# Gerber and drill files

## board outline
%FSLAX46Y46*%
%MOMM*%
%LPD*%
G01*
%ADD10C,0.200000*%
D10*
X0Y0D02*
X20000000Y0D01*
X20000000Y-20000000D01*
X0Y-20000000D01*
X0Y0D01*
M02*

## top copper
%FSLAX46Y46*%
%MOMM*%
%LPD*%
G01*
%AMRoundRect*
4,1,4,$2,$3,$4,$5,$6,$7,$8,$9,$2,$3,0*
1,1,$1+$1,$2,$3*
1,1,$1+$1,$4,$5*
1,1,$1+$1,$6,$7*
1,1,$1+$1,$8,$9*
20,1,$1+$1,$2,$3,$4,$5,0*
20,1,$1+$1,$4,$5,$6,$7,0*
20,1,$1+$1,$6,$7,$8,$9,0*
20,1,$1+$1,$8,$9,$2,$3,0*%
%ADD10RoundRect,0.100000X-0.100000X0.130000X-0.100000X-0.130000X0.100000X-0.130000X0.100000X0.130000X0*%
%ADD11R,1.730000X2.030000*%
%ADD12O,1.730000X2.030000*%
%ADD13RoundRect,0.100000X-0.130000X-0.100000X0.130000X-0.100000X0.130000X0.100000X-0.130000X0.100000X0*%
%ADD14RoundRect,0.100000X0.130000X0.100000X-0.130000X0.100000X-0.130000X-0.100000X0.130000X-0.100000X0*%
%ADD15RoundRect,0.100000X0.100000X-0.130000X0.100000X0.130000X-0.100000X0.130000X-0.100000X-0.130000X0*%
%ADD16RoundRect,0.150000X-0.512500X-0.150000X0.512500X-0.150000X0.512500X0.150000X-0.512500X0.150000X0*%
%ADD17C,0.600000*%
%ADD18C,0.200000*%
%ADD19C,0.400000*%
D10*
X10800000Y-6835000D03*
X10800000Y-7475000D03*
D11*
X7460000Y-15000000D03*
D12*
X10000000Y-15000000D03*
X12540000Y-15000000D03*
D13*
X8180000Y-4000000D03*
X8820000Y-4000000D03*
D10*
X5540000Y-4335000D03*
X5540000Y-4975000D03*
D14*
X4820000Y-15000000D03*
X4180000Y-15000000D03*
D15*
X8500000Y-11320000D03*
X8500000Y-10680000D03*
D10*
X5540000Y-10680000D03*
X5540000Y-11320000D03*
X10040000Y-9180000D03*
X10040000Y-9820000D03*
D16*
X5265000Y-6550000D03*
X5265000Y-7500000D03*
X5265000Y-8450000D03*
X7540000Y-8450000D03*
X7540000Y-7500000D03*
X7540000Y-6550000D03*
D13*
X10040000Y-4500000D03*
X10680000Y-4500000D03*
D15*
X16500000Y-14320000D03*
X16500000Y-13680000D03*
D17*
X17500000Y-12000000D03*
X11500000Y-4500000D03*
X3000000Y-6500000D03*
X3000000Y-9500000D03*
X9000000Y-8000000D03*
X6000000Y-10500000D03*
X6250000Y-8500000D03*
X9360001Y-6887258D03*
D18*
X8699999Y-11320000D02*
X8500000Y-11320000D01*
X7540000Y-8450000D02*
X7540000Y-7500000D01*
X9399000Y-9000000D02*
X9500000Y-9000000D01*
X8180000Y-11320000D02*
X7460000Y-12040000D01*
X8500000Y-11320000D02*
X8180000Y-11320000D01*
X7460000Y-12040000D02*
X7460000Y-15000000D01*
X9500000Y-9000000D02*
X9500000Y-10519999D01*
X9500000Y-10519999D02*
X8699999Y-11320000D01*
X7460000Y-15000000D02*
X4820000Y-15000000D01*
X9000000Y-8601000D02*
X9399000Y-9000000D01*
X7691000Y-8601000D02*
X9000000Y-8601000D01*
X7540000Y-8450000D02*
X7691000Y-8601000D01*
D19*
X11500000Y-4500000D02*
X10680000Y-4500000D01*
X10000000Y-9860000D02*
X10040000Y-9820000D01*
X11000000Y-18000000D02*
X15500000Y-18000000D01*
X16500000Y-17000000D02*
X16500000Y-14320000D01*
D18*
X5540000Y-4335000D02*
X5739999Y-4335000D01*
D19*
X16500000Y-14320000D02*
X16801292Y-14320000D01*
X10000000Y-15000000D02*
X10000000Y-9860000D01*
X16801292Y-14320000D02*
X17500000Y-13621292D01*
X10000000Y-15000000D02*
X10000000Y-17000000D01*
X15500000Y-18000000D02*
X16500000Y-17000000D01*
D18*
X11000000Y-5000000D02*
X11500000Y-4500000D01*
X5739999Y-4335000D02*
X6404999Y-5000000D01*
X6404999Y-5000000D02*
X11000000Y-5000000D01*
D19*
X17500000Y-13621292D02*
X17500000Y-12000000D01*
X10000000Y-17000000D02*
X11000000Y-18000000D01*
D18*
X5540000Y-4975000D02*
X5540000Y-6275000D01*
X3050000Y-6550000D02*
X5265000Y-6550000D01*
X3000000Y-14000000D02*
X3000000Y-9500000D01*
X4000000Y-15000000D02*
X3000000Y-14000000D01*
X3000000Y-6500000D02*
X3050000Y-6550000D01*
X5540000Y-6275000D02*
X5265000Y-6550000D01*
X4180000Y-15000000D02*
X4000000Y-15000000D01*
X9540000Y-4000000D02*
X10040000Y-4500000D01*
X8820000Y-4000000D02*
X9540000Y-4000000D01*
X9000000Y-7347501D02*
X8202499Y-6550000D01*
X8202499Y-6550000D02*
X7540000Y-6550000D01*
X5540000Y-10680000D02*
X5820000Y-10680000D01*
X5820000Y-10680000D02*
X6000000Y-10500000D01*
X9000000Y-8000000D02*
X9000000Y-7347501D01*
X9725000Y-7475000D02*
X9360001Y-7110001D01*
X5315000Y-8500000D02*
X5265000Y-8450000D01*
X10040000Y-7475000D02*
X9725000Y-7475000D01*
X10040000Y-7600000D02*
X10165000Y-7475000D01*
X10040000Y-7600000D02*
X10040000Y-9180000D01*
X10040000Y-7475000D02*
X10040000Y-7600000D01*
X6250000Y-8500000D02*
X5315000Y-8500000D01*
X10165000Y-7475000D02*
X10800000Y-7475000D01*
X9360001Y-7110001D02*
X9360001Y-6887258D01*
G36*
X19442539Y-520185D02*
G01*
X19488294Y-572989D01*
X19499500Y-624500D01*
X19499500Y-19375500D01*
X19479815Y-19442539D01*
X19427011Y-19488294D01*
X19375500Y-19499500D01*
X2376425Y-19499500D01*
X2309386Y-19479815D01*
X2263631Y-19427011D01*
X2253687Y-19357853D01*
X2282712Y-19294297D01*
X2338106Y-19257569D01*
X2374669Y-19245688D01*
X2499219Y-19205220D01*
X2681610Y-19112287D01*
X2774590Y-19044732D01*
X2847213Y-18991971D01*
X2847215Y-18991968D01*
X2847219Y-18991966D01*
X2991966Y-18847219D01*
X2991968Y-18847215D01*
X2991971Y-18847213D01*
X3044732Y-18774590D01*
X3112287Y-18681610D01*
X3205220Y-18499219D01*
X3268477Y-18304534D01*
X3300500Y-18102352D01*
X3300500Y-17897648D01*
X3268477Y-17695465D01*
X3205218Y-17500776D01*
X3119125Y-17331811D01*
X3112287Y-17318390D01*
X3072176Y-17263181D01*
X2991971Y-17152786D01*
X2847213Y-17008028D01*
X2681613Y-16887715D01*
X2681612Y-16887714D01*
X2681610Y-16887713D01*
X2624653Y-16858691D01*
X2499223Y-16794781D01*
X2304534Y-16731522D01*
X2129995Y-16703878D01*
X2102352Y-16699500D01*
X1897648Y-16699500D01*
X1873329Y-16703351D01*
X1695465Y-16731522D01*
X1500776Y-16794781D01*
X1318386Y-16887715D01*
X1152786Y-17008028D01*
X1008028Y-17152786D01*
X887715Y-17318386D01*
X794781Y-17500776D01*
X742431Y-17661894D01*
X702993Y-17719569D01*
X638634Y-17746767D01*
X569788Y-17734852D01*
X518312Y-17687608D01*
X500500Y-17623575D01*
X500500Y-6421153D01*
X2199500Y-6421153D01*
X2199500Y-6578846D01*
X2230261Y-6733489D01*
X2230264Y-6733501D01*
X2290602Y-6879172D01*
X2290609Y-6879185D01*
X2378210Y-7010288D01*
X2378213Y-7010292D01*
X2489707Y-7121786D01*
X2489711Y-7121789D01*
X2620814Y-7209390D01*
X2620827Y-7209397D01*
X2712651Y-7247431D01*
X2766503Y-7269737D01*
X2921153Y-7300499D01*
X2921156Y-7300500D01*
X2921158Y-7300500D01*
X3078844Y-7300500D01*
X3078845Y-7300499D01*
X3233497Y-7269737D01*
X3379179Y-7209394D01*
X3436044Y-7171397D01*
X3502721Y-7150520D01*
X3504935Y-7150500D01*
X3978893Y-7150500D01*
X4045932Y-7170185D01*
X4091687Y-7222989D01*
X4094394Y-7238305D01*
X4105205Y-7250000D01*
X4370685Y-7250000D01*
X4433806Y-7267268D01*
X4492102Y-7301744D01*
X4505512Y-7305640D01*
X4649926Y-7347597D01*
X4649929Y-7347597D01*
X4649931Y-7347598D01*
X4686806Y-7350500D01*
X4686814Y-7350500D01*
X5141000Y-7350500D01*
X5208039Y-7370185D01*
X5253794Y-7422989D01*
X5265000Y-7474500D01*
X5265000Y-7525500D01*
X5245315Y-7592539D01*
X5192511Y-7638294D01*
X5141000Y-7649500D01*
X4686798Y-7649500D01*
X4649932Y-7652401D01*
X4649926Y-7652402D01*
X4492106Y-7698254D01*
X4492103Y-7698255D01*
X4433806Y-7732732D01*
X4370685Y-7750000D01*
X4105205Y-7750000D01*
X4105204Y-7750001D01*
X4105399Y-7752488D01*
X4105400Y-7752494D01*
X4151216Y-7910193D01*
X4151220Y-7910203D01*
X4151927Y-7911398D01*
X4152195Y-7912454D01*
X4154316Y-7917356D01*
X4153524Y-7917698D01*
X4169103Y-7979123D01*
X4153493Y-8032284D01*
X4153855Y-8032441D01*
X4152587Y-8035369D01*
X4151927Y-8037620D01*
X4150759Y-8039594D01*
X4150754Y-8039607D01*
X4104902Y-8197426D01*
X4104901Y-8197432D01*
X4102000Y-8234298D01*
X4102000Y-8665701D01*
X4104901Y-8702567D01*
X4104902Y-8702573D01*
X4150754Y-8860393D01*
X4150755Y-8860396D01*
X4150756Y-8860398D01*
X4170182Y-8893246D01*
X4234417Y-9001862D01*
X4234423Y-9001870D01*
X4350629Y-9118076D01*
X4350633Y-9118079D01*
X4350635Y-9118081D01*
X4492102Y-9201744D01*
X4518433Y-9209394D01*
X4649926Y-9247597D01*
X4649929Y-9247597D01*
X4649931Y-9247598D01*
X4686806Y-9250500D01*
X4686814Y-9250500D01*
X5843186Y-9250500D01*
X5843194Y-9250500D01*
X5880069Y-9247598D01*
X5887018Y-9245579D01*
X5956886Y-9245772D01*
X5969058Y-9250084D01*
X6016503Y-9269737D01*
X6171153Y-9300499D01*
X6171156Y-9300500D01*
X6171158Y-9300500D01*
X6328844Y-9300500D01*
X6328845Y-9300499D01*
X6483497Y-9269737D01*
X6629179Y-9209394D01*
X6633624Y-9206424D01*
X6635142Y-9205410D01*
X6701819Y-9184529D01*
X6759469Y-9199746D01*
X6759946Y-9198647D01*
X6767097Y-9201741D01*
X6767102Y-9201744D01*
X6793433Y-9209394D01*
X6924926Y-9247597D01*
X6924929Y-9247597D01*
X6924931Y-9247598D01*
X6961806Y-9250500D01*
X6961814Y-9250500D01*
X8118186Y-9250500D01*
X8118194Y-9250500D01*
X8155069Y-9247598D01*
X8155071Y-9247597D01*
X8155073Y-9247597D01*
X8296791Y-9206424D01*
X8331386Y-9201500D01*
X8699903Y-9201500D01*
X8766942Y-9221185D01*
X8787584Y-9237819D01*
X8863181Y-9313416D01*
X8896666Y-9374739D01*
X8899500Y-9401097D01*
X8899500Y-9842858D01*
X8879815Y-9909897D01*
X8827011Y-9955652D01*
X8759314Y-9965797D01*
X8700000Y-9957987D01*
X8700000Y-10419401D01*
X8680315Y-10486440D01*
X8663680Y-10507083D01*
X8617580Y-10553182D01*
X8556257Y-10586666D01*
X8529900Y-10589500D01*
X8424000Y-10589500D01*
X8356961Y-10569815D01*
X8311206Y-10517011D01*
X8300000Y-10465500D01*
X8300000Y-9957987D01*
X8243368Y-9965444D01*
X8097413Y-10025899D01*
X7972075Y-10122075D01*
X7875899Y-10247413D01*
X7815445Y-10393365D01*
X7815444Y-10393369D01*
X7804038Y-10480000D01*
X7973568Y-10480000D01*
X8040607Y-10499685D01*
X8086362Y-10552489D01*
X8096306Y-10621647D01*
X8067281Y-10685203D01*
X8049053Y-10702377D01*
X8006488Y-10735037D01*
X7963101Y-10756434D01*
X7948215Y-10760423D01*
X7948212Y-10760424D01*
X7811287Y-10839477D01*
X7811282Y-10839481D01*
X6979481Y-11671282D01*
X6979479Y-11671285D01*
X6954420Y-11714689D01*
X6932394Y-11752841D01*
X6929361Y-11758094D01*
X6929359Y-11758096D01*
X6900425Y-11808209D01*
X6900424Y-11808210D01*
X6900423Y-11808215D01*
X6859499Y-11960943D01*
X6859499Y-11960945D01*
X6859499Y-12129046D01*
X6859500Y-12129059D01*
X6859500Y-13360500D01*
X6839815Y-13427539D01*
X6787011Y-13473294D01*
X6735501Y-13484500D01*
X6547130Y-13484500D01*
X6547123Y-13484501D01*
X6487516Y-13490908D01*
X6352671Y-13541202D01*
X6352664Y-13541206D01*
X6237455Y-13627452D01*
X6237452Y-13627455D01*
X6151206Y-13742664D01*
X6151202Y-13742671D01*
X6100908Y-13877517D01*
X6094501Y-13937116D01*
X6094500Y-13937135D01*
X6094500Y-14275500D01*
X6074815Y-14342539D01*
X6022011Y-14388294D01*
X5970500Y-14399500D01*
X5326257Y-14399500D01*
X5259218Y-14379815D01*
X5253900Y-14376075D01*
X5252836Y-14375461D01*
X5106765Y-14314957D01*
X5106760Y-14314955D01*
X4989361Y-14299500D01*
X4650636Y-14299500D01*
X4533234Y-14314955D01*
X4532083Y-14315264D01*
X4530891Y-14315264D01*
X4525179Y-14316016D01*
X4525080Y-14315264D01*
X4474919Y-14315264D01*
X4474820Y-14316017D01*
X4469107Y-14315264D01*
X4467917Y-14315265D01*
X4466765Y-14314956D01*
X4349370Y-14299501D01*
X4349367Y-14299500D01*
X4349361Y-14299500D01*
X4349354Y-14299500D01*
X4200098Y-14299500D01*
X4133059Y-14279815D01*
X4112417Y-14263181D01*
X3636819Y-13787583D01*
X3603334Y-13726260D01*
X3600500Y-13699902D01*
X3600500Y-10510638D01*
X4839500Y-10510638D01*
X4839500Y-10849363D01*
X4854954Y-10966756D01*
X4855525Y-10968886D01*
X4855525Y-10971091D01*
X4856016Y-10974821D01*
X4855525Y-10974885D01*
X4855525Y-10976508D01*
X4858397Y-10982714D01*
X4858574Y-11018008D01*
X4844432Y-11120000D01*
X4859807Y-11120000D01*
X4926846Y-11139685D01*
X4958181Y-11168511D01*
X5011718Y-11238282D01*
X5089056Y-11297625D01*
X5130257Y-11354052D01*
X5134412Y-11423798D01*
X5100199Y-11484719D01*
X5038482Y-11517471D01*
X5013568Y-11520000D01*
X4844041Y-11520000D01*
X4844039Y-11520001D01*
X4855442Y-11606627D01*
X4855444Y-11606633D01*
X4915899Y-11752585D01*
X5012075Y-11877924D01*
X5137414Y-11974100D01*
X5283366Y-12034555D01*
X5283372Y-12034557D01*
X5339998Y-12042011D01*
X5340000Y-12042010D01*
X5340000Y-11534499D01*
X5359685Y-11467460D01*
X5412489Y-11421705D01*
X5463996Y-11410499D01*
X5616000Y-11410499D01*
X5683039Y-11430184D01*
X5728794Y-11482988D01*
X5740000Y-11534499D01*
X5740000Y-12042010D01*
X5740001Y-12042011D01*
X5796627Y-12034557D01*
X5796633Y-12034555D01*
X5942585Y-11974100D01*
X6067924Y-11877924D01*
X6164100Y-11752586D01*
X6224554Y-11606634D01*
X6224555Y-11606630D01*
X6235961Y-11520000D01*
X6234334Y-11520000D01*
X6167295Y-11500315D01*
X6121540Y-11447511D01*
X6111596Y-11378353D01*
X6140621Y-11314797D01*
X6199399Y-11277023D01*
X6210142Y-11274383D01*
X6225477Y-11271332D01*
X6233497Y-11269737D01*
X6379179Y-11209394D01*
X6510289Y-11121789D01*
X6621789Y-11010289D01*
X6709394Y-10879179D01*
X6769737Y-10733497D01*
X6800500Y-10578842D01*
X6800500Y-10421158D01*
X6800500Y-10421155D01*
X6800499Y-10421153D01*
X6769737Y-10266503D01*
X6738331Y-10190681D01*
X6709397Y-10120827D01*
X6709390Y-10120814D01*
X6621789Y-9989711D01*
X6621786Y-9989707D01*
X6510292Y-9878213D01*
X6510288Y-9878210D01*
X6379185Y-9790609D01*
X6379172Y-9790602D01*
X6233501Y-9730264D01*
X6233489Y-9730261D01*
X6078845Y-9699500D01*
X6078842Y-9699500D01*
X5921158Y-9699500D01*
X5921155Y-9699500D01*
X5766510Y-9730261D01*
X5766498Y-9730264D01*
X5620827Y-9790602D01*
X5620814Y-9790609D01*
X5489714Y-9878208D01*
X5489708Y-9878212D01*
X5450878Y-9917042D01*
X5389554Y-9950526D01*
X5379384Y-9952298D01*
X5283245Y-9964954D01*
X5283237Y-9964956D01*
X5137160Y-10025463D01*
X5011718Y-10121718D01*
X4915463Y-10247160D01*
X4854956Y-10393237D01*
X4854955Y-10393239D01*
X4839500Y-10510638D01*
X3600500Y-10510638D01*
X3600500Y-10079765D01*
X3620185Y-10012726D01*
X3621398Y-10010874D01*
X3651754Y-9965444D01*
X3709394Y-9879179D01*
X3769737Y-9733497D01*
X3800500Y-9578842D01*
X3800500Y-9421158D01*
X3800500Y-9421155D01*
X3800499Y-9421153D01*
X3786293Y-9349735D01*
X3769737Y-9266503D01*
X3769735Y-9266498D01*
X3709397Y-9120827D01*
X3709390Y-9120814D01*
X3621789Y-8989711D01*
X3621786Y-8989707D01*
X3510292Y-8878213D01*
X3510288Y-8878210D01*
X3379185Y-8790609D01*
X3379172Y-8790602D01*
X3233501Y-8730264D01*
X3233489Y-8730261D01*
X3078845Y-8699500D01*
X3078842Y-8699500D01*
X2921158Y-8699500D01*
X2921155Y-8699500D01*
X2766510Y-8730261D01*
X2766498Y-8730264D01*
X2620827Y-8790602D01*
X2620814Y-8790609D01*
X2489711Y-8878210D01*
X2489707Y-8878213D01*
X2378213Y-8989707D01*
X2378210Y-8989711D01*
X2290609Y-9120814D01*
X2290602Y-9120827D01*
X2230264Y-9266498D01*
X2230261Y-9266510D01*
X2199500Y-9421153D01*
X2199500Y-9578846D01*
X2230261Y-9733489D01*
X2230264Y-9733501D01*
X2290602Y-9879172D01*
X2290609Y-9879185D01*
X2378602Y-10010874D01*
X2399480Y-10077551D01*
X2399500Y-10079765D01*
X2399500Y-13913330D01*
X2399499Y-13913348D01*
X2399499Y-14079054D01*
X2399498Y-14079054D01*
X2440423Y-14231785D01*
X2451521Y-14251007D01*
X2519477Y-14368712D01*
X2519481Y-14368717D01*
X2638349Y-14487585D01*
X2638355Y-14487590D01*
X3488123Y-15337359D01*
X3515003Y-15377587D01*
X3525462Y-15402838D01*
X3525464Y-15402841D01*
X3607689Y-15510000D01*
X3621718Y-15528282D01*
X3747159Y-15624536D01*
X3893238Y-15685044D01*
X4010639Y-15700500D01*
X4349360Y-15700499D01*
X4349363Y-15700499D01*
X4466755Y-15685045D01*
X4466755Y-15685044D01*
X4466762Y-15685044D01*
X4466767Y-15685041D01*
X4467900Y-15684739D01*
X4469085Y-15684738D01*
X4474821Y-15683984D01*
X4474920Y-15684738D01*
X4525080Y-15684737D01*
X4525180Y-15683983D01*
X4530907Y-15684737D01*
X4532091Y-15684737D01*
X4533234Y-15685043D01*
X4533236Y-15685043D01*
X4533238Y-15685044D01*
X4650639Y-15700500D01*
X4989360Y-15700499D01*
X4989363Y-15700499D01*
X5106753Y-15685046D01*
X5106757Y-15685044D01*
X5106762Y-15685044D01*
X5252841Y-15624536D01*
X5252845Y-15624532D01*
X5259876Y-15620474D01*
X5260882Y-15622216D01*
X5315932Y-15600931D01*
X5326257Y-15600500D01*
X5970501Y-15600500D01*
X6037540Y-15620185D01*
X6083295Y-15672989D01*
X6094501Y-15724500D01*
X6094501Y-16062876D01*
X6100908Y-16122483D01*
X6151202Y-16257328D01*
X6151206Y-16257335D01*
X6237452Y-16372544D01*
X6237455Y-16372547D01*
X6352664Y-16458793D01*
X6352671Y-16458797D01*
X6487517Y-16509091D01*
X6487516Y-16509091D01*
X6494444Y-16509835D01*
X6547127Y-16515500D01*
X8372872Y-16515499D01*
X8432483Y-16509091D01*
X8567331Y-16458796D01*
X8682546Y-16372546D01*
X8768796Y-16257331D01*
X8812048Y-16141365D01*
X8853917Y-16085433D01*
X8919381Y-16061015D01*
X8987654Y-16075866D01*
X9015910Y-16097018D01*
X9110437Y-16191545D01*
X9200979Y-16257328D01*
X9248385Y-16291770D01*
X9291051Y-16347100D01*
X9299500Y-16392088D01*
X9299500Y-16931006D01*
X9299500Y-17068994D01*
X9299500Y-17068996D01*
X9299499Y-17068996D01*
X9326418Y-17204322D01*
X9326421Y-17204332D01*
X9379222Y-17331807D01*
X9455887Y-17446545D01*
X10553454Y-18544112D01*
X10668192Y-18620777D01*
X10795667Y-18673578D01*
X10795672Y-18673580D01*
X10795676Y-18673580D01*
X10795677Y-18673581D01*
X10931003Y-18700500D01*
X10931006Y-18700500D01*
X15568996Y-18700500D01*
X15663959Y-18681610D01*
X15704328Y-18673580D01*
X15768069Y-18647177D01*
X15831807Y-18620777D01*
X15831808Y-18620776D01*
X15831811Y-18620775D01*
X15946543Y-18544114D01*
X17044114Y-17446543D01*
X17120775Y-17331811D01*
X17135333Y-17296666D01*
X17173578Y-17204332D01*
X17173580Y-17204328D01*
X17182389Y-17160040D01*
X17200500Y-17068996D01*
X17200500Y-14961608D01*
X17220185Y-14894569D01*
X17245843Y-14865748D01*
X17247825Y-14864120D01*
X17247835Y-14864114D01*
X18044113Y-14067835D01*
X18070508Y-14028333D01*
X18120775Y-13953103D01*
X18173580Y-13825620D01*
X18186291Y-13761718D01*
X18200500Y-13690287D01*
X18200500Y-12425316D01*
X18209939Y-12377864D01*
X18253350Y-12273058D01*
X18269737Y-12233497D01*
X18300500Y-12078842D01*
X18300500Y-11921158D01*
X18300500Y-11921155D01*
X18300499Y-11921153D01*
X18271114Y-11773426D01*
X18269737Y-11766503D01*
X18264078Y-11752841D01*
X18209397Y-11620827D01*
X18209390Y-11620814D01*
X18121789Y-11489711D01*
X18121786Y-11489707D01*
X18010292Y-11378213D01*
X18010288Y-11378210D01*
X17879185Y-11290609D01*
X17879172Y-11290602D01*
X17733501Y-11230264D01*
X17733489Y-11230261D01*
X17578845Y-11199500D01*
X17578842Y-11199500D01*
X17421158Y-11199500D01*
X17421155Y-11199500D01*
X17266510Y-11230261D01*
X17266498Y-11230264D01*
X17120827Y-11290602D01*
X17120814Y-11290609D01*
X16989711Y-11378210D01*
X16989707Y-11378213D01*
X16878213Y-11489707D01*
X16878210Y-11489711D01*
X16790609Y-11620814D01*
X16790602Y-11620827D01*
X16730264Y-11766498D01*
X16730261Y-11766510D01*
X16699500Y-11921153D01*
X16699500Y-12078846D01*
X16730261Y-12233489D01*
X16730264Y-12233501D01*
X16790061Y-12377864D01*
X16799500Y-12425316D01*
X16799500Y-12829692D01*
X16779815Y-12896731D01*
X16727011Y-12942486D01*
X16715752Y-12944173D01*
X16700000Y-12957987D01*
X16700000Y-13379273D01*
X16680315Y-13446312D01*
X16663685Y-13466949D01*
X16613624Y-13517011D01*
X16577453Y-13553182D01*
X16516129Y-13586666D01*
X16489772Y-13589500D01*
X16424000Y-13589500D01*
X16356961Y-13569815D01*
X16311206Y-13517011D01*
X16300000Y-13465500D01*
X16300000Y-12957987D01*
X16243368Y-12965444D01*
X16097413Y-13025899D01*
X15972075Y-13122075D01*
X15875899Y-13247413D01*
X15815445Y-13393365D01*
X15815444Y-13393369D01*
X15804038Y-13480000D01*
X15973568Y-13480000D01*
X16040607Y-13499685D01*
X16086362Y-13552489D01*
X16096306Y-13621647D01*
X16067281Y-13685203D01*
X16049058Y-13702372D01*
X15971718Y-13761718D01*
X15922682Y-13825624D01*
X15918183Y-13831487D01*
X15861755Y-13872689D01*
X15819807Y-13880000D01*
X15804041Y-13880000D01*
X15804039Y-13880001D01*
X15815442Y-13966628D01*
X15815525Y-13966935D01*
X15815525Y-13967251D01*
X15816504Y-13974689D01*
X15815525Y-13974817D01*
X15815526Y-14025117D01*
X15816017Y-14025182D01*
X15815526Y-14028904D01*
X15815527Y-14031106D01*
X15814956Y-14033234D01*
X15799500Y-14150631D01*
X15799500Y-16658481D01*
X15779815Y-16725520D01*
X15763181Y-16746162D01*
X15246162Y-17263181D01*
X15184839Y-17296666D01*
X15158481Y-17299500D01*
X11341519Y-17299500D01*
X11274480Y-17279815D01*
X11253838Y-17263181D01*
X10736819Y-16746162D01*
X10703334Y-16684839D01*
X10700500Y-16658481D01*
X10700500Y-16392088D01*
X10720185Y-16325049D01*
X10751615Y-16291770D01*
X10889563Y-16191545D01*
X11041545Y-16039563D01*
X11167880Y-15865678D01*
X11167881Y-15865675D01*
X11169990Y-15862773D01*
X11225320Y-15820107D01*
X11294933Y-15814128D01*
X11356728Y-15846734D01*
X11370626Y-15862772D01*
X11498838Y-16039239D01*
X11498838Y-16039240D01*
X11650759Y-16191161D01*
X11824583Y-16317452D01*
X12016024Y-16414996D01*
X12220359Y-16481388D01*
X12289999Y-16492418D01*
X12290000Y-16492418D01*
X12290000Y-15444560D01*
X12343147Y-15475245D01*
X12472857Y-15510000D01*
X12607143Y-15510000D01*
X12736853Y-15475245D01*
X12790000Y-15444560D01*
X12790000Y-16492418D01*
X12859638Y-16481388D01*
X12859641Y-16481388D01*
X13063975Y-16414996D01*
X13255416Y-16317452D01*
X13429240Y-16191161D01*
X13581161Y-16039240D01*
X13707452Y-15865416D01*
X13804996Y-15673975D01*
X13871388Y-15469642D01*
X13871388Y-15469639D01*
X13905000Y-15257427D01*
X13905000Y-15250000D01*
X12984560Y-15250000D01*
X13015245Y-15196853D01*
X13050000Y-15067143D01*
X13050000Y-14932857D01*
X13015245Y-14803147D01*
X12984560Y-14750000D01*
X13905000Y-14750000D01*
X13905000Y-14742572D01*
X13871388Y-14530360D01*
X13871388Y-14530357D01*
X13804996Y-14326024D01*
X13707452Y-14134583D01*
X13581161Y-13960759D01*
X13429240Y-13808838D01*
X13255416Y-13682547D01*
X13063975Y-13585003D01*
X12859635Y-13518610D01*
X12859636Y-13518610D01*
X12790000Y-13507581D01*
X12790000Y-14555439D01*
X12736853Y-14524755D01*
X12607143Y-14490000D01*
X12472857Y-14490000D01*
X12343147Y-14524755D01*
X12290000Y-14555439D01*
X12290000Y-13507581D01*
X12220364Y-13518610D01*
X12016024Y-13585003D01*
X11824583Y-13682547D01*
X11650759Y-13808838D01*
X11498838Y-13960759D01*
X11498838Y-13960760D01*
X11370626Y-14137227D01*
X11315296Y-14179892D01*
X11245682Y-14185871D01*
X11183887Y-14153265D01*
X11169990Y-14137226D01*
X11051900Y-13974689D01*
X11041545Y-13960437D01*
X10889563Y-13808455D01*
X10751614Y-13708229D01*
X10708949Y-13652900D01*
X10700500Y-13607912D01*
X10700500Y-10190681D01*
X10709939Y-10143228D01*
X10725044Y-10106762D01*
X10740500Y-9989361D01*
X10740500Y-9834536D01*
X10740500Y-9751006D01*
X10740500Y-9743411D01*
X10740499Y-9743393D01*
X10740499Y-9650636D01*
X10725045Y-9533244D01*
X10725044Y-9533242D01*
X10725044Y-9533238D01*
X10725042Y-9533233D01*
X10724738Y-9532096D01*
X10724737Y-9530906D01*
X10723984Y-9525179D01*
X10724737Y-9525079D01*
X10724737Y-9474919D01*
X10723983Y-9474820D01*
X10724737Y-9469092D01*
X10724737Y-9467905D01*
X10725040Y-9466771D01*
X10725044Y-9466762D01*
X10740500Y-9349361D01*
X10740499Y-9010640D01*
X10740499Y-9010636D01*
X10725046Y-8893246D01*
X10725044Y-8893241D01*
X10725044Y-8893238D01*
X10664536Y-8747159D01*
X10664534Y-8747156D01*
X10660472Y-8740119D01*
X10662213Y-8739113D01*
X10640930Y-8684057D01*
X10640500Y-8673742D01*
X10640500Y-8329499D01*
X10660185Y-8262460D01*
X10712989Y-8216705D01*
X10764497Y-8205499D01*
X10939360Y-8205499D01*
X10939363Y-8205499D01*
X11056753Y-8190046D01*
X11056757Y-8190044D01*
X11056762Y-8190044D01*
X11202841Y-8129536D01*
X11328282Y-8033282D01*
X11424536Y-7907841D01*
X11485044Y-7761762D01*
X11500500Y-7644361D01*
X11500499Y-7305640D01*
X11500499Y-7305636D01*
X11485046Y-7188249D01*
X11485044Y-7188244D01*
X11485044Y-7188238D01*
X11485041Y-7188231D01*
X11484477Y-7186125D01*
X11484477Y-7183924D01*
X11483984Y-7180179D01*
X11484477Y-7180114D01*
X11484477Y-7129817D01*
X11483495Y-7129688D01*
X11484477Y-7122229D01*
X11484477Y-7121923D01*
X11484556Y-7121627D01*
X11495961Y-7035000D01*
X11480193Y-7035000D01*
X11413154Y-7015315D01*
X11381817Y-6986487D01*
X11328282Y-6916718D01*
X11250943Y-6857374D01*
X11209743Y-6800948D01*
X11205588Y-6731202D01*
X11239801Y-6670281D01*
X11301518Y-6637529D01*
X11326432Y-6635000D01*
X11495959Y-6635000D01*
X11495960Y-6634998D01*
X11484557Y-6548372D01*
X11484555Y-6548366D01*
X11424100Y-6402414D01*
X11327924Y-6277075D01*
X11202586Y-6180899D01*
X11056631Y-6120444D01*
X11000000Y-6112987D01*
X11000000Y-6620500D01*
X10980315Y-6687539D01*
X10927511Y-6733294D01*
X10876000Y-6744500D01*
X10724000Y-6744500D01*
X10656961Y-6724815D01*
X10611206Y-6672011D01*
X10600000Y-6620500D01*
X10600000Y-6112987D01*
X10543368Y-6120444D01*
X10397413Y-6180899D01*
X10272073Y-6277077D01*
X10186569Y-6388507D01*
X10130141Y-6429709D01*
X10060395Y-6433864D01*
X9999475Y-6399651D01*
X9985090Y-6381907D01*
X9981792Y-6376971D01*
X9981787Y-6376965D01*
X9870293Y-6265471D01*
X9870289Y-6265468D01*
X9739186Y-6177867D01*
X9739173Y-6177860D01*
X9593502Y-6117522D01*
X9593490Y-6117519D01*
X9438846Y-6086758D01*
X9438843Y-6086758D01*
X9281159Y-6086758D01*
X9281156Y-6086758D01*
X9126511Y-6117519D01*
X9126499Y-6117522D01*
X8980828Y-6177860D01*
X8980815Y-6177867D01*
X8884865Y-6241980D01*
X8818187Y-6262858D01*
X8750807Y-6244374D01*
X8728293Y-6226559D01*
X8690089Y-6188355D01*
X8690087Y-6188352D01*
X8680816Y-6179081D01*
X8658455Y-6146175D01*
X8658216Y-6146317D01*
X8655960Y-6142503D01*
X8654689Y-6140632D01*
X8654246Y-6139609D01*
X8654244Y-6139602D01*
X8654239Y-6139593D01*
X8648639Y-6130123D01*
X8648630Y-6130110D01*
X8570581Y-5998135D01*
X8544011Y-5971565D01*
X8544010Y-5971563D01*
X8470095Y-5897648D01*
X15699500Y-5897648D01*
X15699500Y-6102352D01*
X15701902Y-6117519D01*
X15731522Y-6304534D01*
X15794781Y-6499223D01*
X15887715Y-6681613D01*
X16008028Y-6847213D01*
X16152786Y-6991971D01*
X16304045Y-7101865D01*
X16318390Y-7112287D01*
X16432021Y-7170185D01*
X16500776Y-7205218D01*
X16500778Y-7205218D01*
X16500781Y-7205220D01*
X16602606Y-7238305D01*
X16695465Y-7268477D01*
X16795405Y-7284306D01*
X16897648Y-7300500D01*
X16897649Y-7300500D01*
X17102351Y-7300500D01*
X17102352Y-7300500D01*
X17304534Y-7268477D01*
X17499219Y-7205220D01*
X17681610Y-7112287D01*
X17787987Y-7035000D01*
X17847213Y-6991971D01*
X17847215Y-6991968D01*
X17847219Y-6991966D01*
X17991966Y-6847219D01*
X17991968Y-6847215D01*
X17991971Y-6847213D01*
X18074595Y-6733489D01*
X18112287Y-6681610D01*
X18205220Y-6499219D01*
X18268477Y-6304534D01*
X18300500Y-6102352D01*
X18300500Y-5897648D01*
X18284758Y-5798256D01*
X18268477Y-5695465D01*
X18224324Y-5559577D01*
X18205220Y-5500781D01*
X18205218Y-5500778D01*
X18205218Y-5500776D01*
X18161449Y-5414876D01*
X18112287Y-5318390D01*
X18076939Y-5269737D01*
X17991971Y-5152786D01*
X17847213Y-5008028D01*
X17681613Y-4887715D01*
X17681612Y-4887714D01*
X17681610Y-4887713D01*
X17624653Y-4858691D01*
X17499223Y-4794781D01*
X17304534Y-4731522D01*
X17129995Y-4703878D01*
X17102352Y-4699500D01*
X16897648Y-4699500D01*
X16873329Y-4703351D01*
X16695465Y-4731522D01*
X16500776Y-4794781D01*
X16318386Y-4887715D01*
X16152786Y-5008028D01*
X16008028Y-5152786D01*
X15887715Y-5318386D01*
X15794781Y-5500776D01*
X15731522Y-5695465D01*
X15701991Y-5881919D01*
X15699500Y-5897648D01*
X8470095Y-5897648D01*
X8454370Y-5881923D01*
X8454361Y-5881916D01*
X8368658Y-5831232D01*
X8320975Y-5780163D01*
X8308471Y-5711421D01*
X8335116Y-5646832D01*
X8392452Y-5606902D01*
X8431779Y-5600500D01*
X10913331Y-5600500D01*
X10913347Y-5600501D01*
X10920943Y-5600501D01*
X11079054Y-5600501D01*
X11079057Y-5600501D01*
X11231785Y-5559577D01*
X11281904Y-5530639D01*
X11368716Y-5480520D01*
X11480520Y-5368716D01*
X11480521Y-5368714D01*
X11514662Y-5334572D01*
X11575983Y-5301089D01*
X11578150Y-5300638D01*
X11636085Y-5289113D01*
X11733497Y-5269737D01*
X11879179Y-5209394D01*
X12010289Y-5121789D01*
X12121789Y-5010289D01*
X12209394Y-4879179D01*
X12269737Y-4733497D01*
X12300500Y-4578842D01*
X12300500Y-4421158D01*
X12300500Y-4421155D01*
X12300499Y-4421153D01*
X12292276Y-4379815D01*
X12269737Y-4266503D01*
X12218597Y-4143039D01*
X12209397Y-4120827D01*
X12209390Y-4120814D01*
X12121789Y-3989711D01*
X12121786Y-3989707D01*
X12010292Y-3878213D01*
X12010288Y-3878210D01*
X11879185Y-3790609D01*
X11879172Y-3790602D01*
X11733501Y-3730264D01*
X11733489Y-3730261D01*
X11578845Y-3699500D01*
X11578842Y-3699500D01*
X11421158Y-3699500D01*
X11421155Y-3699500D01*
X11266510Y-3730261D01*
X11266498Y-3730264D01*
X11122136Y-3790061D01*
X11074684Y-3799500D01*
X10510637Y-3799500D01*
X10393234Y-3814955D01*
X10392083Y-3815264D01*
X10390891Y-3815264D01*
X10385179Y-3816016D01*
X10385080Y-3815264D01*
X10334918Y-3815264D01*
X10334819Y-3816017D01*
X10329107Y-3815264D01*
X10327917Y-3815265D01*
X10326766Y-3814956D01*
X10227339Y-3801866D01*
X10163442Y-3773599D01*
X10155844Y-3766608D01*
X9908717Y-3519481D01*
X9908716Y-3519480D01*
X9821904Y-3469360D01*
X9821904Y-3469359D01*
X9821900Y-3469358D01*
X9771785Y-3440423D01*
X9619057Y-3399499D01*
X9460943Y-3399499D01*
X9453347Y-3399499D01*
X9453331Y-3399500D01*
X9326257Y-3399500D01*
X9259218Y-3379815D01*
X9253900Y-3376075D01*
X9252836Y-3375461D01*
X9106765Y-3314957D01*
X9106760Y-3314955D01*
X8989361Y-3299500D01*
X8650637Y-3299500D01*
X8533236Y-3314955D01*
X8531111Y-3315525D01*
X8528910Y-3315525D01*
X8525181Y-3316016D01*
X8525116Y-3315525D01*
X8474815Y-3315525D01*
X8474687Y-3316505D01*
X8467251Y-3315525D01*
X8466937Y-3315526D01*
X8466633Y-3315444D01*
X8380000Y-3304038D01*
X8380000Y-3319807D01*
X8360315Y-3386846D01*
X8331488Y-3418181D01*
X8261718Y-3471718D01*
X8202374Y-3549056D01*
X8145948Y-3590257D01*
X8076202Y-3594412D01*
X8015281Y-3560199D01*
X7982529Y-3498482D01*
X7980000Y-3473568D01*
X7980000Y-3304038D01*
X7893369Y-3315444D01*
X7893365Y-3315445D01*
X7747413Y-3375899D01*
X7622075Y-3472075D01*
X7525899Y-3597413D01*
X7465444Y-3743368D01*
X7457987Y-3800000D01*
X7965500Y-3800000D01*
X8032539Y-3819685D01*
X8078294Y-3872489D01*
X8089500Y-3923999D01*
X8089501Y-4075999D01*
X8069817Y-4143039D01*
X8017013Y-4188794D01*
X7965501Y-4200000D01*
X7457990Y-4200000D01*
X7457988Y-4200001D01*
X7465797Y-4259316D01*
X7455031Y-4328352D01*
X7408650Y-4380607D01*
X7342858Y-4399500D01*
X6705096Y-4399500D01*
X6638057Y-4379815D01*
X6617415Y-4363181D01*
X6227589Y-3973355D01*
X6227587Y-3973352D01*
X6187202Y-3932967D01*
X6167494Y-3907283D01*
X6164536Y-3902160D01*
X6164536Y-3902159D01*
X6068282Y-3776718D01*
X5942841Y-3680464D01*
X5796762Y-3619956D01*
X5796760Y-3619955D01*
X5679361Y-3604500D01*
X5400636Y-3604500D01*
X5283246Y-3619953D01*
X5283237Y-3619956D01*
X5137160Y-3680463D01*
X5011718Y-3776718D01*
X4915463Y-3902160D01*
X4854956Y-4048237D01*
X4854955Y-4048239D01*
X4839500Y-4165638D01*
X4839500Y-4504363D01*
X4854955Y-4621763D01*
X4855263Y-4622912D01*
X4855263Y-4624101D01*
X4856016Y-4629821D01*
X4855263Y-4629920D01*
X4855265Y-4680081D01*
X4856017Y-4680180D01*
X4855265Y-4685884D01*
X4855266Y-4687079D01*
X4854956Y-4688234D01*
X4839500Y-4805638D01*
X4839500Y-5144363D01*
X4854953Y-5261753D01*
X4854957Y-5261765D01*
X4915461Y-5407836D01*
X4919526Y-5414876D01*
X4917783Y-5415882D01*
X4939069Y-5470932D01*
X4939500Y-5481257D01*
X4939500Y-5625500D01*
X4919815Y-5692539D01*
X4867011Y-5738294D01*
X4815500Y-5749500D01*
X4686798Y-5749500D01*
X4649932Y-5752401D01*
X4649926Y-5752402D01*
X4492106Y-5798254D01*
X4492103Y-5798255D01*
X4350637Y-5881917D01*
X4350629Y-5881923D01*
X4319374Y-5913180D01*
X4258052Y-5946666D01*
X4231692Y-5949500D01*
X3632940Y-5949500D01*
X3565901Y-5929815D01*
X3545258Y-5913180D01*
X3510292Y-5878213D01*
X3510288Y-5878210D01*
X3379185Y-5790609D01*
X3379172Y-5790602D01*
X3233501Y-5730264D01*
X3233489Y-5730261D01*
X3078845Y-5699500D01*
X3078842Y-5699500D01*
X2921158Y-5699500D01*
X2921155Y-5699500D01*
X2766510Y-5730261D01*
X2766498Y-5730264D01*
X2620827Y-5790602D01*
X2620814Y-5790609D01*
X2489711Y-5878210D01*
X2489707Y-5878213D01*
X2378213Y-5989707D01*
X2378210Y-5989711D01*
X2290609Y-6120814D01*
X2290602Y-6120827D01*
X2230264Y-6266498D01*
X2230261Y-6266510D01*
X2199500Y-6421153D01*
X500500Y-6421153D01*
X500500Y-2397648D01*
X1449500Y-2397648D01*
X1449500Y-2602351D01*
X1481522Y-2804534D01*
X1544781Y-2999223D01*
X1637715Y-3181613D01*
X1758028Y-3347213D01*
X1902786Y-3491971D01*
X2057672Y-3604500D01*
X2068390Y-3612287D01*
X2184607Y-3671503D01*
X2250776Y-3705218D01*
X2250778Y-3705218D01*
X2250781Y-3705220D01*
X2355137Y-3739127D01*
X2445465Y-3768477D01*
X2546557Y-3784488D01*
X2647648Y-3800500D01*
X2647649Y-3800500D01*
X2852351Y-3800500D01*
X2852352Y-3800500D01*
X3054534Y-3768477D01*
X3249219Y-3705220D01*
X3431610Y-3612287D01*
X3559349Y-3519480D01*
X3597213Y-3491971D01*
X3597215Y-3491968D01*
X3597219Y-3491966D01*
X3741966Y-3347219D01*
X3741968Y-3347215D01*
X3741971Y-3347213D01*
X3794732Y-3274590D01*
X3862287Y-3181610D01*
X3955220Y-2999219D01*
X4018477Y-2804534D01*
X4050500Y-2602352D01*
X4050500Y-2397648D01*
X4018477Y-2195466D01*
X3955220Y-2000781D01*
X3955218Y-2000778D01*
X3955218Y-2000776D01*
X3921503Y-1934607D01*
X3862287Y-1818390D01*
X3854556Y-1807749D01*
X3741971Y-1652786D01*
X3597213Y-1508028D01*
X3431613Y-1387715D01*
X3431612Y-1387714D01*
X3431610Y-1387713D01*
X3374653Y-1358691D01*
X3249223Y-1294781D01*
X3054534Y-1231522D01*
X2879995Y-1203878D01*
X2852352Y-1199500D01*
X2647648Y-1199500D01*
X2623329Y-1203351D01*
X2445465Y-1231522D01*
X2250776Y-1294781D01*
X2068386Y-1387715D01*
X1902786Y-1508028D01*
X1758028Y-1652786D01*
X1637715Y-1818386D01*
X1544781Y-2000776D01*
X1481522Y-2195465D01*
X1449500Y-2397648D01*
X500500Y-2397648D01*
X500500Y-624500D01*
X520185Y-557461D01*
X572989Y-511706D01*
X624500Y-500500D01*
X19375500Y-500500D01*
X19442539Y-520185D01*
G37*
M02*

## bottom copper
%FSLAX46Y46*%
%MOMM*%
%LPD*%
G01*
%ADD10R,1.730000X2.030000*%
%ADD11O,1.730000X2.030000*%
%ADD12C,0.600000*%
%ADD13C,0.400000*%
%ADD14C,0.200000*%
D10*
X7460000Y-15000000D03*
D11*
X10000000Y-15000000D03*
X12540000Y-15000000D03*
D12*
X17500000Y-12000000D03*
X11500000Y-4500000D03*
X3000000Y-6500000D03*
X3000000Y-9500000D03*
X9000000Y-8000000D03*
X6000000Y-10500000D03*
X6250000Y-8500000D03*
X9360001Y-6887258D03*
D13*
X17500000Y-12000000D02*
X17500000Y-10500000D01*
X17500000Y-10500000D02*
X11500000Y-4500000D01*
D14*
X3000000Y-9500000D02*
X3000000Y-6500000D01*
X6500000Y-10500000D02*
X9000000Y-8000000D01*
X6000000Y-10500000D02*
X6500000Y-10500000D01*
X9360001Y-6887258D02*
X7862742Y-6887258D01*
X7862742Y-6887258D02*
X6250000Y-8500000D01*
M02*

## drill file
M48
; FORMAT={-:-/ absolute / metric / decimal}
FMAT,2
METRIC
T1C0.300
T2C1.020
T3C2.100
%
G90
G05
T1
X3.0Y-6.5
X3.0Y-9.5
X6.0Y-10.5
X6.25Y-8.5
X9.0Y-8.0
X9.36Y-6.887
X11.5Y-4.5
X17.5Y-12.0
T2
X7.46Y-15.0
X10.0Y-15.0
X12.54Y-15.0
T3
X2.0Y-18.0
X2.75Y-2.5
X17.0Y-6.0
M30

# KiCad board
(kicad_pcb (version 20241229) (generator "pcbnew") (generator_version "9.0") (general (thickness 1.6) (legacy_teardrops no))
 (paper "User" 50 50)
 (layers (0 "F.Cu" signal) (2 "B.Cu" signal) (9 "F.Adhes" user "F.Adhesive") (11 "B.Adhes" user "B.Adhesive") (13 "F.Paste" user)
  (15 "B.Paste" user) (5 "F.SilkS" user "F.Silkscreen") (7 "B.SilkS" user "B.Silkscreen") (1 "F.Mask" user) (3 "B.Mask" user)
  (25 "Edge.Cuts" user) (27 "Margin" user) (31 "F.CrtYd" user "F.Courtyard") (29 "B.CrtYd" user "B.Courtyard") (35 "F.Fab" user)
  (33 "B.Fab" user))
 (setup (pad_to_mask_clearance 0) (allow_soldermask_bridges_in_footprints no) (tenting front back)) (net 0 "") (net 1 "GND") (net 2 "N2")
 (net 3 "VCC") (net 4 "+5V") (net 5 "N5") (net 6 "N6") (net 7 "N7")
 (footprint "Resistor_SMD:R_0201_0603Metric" (layer "F.Cu") (at 10.8 7.155 -90)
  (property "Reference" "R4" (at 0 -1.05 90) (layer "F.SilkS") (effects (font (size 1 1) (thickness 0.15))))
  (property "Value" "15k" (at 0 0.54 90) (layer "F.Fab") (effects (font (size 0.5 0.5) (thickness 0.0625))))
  (pad "" smd roundrect (at -0.345 0 270) (size 0.318 0.36) (layers "F.Paste") (roundrect_rratio 0.25))
  (pad "" smd roundrect (at 0.345 0 270) (size 0.318 0.36) (layers "F.Paste") (roundrect_rratio 0.25))
  (pad "1" smd roundrect (at -0.32 0 270) (size 0.46 0.4) (layers "F.Cu" "F.Mask") (roundrect_rratio 0.25) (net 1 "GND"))
  (pad "2" smd roundrect (at 0.32 0 270) (size 0.46 0.4) (layers "F.Cu" "F.Mask") (roundrect_rratio 0.25) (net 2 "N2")))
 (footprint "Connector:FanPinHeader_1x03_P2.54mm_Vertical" (layer "F.Cu") (at 7.46 15)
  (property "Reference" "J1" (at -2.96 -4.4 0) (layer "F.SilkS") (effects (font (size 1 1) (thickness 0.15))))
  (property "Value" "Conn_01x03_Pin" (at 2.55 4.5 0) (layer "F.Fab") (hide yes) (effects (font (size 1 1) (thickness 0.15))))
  (pad "1" thru_hole rect (at 0 0 90) (size 2.03 1.73) (drill 1.02) (layers "*.Cu" "*.Mask") (remove_unused_layers no) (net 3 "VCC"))
  (pad "2" thru_hole oval (at 2.54 0 90) (size 2.03 1.73) (drill 1.02) (layers "*.Cu" "*.Mask") (remove_unused_layers no) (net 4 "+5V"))
  (pad "3" thru_hole oval (at 5.08 0 90) (size 2.03 1.73) (drill 1.02) (layers "*.Cu" "*.Mask") (remove_unused_layers no) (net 1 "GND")))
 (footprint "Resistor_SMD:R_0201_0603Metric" (layer "F.Cu") (at 8.5 4)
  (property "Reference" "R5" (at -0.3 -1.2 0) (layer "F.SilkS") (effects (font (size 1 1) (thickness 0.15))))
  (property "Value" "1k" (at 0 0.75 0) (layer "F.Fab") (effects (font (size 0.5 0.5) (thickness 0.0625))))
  (pad "" smd roundrect (at -0.345 0) (size 0.318 0.36) (layers "F.Paste") (roundrect_rratio 0.25))
  (pad "" smd roundrect (at 0.345 0) (size 0.318 0.36) (layers "F.Paste") (roundrect_rratio 0.25))
  (pad "1" smd roundrect (at -0.32 0) (size 0.46 0.4) (layers "F.Cu" "F.Mask") (roundrect_rratio 0.25) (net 1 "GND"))
  (pad "2" smd roundrect (at 0.32 0) (size 0.46 0.4) (layers "F.Cu" "F.Mask") (roundrect_rratio 0.25) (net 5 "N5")))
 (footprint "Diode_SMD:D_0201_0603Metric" (layer "F.Cu") (at 5.54 4.655 -90)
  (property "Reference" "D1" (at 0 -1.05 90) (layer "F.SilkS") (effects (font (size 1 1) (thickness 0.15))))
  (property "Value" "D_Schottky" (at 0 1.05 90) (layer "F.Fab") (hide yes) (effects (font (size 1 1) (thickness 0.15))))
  (pad "" smd roundrect (at -0.345 0 270) (size 0.318 0.36) (layers "F.Paste") (roundrect_rratio 0.25))
  (pad "" smd roundrect (at 0.345 0 270) (size 0.318 0.36) (layers "F.Paste") (roundrect_rratio 0.25))
  (pad "1" smd roundrect (at -0.32 0 270) (size 0.46 0.4) (layers "F.Cu" "F.Mask") (roundrect_rratio 0.25) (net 4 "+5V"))
  (pad "2" smd roundrect (at 0.32 0 270) (size 0.46 0.4) (layers "F.Cu" "F.Mask") (roundrect_rratio 0.25) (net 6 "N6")))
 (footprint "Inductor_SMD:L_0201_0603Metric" (layer "F.Cu") (at 4.5 15 180)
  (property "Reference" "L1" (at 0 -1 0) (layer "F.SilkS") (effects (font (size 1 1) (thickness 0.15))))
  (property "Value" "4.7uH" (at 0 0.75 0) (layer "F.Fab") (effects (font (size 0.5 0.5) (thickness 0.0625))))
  (pad "" smd roundrect (at -0.345 0 180) (size 0.318 0.36) (layers "F.Paste") (roundrect_rratio 0.25))
  (pad "" smd roundrect (at 0.345 0 180) (size 0.318 0.36) (layers "F.Paste") (roundrect_rratio 0.25))
  (pad "1" smd roundrect (at -0.32 0 180) (size 0.46 0.4) (layers "F.Cu" "F.Mask") (roundrect_rratio 0.25) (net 3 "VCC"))
  (pad "2" smd roundrect (at 0.32 0 180) (size 0.46 0.4) (layers "F.Cu" "F.Mask") (roundrect_rratio 0.25) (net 6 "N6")))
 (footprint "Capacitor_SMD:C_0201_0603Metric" (layer "F.Cu") (at 8.5 11 90)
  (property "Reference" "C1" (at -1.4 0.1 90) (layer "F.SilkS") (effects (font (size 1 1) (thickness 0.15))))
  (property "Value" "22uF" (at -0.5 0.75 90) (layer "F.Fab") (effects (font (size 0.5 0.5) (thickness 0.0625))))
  (pad "" smd roundrect (at -0.345 0 90) (size 0.318 0.36) (layers "F.Paste") (roundrect_rratio 0.25))
  (pad "" smd roundrect (at 0.345 0 90) (size 0.318 0.36) (layers "F.Paste") (roundrect_rratio 0.25))
  (pad "1" smd roundrect (at -0.32 0 90) (size 0.46 0.4) (layers "F.Cu" "F.Mask") (roundrect_rratio 0.25) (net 3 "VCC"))
  (pad "2" smd roundrect (at 0.32 0 90) (size 0.46 0.4) (layers "F.Cu" "F.Mask") (roundrect_rratio 0.25) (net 1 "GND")))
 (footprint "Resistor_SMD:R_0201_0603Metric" (layer "F.Cu") (at 5.54 11 -90)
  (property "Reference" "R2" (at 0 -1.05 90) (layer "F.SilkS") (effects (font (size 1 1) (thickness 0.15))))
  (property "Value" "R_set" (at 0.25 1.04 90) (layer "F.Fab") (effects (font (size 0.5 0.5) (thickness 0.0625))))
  (pad "" smd roundrect (at -0.345 0 270) (size 0.318 0.36) (layers "F.Paste") (roundrect_rratio 0.25))
  (pad "" smd roundrect (at 0.345 0 270) (size 0.318 0.36) (layers "F.Paste") (roundrect_rratio 0.25))
  (pad "1" smd roundrect (at -0.32 0 270) (size 0.46 0.4) (layers "F.Cu" "F.Mask") (roundrect_rratio 0.25) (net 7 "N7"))
  (pad "2" smd roundrect (at 0.32 0 270) (size 0.46 0.4) (layers "F.Cu" "F.Mask") (roundrect_rratio 0.25) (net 1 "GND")))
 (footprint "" (layer "F.Cu") (at 2 18)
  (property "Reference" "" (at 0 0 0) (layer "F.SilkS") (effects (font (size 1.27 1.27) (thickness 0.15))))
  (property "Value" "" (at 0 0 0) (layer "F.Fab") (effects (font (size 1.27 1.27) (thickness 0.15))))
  (pad "" np_thru_hole circle (at 0 0) (size 2.1 2.1) (drill 2.1) (layers "*.Cu" "*.Mask")))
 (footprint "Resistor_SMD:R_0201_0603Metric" (layer "F.Cu") (at 10.04 9.5 -90)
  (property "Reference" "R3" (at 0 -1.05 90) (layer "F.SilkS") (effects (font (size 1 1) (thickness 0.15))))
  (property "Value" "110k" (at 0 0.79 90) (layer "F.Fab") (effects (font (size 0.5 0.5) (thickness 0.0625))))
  (pad "" smd roundrect (at -0.345 0 270) (size 0.318 0.36) (layers "F.Paste") (roundrect_rratio 0.25))
  (pad "" smd roundrect (at 0.345 0 270) (size 0.318 0.36) (layers "F.Paste") (roundrect_rratio 0.25))
  (pad "1" smd roundrect (at -0.32 0 270) (size 0.46 0.4) (layers "F.Cu" "F.Mask") (roundrect_rratio 0.25) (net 2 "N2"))
  (pad "2" smd roundrect (at 0.32 0 270) (size 0.46 0.4) (layers "F.Cu" "F.Mask") (roundrect_rratio 0.25) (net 4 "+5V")))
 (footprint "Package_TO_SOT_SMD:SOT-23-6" (layer "F.Cu") (at 6.4025 7.5)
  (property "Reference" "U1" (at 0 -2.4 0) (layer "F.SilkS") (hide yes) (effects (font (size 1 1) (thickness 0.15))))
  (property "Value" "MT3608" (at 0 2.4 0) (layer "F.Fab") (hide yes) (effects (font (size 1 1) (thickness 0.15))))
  (pad "1" smd roundrect (at -1.1375 -0.95) (size 1.325 0.6) (layers "F.Cu" "F.Mask" "F.Paste") (roundrect_rratio 0.25) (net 6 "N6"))
  (pad "2" smd roundrect (at -1.1375 0) (size 1.325 0.6) (layers "F.Cu" "F.Mask" "F.Paste") (roundrect_rratio 0.25) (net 1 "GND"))
  (pad "3" smd roundrect (at -1.1375 0.95) (size 1.325 0.6) (layers "F.Cu" "F.Mask" "F.Paste") (roundrect_rratio 0.25) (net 2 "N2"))
  (pad "4" smd roundrect (at 1.1375 0.95) (size 1.325 0.6) (layers "F.Cu" "F.Mask" "F.Paste") (roundrect_rratio 0.25) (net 3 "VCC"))
  (pad "5" smd roundrect (at 1.1375 0) (size 1.325 0.6) (layers "F.Cu" "F.Mask" "F.Paste") (roundrect_rratio 0.25) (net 3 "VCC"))
  (pad "6" smd roundrect (at 1.1375 -0.95) (size 1.325 0.6) (layers "F.Cu" "F.Mask" "F.Paste") (roundrect_rratio 0.25) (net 7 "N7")))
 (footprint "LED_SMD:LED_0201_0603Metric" (layer "F.Cu") (at 10.36 4.5)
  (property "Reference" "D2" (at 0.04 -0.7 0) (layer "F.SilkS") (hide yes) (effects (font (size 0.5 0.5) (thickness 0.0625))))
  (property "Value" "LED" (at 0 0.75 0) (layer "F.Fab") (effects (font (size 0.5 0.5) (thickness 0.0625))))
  (pad "" smd roundrect (at -0.345 0) (size 0.318 0.36) (layers "F.Paste") (roundrect_rratio 0.25))
  (pad "" smd roundrect (at 0.345 0) (size 0.318 0.36) (layers "F.Paste") (roundrect_rratio 0.25))
  (pad "1" smd roundrect (at -0.32 0) (size 0.46 0.4) (layers "F.Cu" "F.Mask") (roundrect_rratio 0.25) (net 5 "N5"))
  (pad "2" smd roundrect (at 0.32 0) (size 0.46 0.4) (layers "F.Cu" "F.Mask") (roundrect_rratio 0.25) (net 4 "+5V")))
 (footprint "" (layer "F.Cu") (at 2.75 2.5)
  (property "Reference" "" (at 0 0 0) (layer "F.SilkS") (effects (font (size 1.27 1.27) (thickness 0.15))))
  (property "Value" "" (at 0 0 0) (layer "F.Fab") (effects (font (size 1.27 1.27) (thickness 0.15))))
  (pad "" np_thru_hole circle (at 0 0) (size 2.1 2.1) (drill 2.1) (layers "*.Cu" "*.Mask")))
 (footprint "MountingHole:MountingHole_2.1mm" (layer "F.Cu") (at 17 6)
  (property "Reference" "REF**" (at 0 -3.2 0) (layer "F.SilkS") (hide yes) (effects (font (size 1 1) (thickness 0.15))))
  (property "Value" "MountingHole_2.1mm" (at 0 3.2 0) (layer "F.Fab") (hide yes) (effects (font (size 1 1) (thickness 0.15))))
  (pad "" np_thru_hole circle (at 0 0) (size 2.1 2.1) (drill 2.1) (layers "*.Cu" "*.Mask")))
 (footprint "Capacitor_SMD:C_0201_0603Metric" (layer "F.Cu") (at 16.5 14 90)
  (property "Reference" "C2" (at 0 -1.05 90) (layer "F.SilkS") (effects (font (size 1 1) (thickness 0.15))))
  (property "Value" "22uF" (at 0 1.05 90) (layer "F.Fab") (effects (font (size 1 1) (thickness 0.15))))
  (pad "" smd roundrect (at -0.345 0 90) (size 0.318 0.36) (layers "F.Paste") (roundrect_rratio 0.25))
  (pad "" smd roundrect (at 0.345 0 90) (size 0.318 0.36) (layers "F.Paste") (roundrect_rratio 0.25))
  (pad "1" smd roundrect (at -0.32 0 90) (size 0.46 0.4) (layers "F.Cu" "F.Mask") (roundrect_rratio 0.25) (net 4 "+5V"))
  (pad "2" smd roundrect (at 0.32 0 90) (size 0.46 0.4) (layers "F.Cu" "F.Mask") (roundrect_rratio 0.25) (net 1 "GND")))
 (gr_rect (start 0 0) (end 20 20) (stroke (width 0.2) (type solid)) (fill no) (layer "Edge.Cuts"))
 (segment (start 8.699999 11.32) (end 8.5 11.32) (width 0.2) (layer "F.Cu") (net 3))
 (segment (start 7.54 8.45) (end 7.54 7.5) (width 0.2) (layer "F.Cu") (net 3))
 (segment (start 9.399 9) (end 9.5 9) (width 0.2) (layer "F.Cu") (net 3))
 (segment (start 8.18 11.32) (end 7.46 12.04) (width 0.2) (layer "F.Cu") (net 3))
 (segment (start 8.5 11.32) (end 8.18 11.32) (width 0.2) (layer "F.Cu") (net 3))
 (segment (start 7.46 12.04) (end 7.46 15) (width 0.2) (layer "F.Cu") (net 3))
 (segment (start 9.5 9) (end 9.5 10.519999) (width 0.2) (layer "F.Cu") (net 3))
 (segment (start 9.5 10.519999) (end 8.699999 11.32) (width 0.2) (layer "F.Cu") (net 3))
 (segment (start 7.46 15) (end 4.82 15) (width 0.2) (layer "F.Cu") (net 3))
 (segment (start 9 8.601) (end 9.399 9) (width 0.2) (layer "F.Cu") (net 3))
 (segment (start 7.691 8.601) (end 9 8.601) (width 0.2) (layer "F.Cu") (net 3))
 (segment (start 7.54 8.45) (end 7.691 8.601) (width 0.2) (layer "F.Cu") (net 3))
 (segment (start 11.5 4.5) (end 10.68 4.5) (width 0.4) (layer "F.Cu") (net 4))
 (segment (start 10 9.86) (end 10.04 9.82) (width 0.4) (layer "F.Cu") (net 4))
 (segment (start 11 18) (end 15.5 18) (width 0.4) (layer "F.Cu") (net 4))
 (segment (start 16.5 17) (end 16.5 14.32) (width 0.4) (layer "F.Cu") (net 4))
 (segment (start 5.54 4.335) (end 5.739999 4.335) (width 0.2) (layer "F.Cu") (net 4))
 (segment (start 16.5 14.32) (end 16.801292 14.32) (width 0.4) (layer "F.Cu") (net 4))
 (segment (start 10 15) (end 10 9.86) (width 0.4) (layer "F.Cu") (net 4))
 (segment (start 16.801292 14.32) (end 17.5 13.621292) (width 0.4) (layer "F.Cu") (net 4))
 (segment (start 10 15) (end 10 17) (width 0.4) (layer "F.Cu") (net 4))
 (segment (start 15.5 18) (end 16.5 17) (width 0.4) (layer "F.Cu") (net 4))
 (segment (start 11 5) (end 11.5 4.5) (width 0.2) (layer "F.Cu") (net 4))
 (segment (start 5.739999 4.335) (end 6.404999 5) (width 0.2) (layer "F.Cu") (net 4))
 (segment (start 6.404999 5) (end 11 5) (width 0.2) (layer "F.Cu") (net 4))
 (segment (start 17.5 13.621292) (end 17.5 12) (width 0.4) (layer "F.Cu") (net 4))
 (segment (start 10 17) (end 11 18) (width 0.4) (layer "F.Cu") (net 4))
 (via (at 17.5 12) (size 0.6) (drill 0.3) (layers "F.Cu" "B.Cu") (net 4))
 (via (at 11.5 4.5) (size 0.6) (drill 0.3) (layers "F.Cu" "B.Cu") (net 4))
 (segment (start 17.5 12) (end 17.5 10.5) (width 0.4) (layer "B.Cu") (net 4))
 (segment (start 17.5 10.5) (end 11.5 4.5) (width 0.4) (layer "B.Cu") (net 4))
 (segment (start 5.54 4.975) (end 5.54 6.275) (width 0.2) (layer "F.Cu") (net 6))
 (segment (start 3.05 6.55) (end 5.265 6.55) (width 0.2) (layer "F.Cu") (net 6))
 (segment (start 3 14) (end 3 9.5) (width 0.2) (layer "F.Cu") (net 6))
 (segment (start 4 15) (end 3 14) (width 0.2) (layer "F.Cu") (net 6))
 (segment (start 3 6.5) (end 3.05 6.55) (width 0.2) (layer "F.Cu") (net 6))
 (segment (start 5.54 6.275) (end 5.265 6.55) (width 0.2) (layer "F.Cu") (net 6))
 (segment (start 4.18 15) (end 4 15) (width 0.2) (layer "F.Cu") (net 6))
 (via (at 3 6.5) (size 0.6) (drill 0.3) (layers "F.Cu" "B.Cu") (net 6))
 (via (at 3 9.5) (size 0.6) (drill 0.3) (layers "F.Cu" "B.Cu") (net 6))
 (segment (start 3 9.5) (end 3 6.5) (width 0.2) (layer "B.Cu") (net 6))
 (segment (start 9.54 4) (end 10.04 4.5) (width 0.2) (layer "F.Cu") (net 5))
 (segment (start 8.82 4) (end 9.54 4) (width 0.2) (layer "F.Cu") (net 5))
 (segment (start 9 7.347501) (end 8.202499 6.55) (width 0.2) (layer "F.Cu") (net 7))
 (segment (start 8.202499 6.55) (end 7.54 6.55) (width 0.2) (layer "F.Cu") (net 7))
 (segment (start 5.54 10.68) (end 5.82 10.68) (width 0.2) (layer "F.Cu") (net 7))
 (segment (start 5.82 10.68) (end 6 10.5) (width 0.2) (layer "F.Cu") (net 7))
 (segment (start 9 8) (end 9 7.347501) (width 0.2) (layer "F.Cu") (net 7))
 (via (at 9 8) (size 0.6) (drill 0.3) (layers "F.Cu" "B.Cu") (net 7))
 (via (at 6 10.5) (size 0.6) (drill 0.3) (layers "F.Cu" "B.Cu") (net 7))
 (segment (start 6.5 10.5) (end 9 8) (width 0.2) (layer "B.Cu") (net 7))
 (segment (start 6 10.5) (end 6.5 10.5) (width 0.2) (layer "B.Cu") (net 7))
 (segment (start 9.725 7.475) (end 9.360001 7.110001) (width 0.2) (layer "F.Cu") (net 2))
 (segment (start 5.315 8.5) (end 5.265 8.45) (width 0.2) (layer "F.Cu") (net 2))
 (segment (start 10.04 7.475) (end 9.725 7.475) (width 0.2) (layer "F.Cu") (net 2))
 (segment (start 10.04 7.6) (end 10.165 7.475) (width 0.2) (layer "F.Cu") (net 2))
 (segment (start 10.04 7.6) (end 10.04 9.18) (width 0.2) (layer "F.Cu") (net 2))
 (segment (start 10.04 7.475) (end 10.04 7.6) (width 0.2) (layer "F.Cu") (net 2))
 (segment (start 6.25 8.5) (end 5.315 8.5) (width 0.2) (layer "F.Cu") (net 2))
 (segment (start 10.165 7.475) (end 10.8 7.475) (width 0.2) (layer "F.Cu") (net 2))
 (segment (start 9.360001 7.110001) (end 9.360001 6.887258) (width 0.2) (layer "F.Cu") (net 2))
 (via (at 6.25 8.5) (size 0.6) (drill 0.3) (layers "F.Cu" "B.Cu") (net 2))
 (via (at 9.360001 6.887258) (size 0.6) (drill 0.3) (layers "F.Cu" "B.Cu") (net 2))
 (segment (start 9.360001 6.887258) (end 7.862742 6.887258) (width 0.2) (layer "B.Cu") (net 2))
 (segment (start 7.862742 6.887258) (end 6.25 8.5) (width 0.2) (layer "B.Cu") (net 2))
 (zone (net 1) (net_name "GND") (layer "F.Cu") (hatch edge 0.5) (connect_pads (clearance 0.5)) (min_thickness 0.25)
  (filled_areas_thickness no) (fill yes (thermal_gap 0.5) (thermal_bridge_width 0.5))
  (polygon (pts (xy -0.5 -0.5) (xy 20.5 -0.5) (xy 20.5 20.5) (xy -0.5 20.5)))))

